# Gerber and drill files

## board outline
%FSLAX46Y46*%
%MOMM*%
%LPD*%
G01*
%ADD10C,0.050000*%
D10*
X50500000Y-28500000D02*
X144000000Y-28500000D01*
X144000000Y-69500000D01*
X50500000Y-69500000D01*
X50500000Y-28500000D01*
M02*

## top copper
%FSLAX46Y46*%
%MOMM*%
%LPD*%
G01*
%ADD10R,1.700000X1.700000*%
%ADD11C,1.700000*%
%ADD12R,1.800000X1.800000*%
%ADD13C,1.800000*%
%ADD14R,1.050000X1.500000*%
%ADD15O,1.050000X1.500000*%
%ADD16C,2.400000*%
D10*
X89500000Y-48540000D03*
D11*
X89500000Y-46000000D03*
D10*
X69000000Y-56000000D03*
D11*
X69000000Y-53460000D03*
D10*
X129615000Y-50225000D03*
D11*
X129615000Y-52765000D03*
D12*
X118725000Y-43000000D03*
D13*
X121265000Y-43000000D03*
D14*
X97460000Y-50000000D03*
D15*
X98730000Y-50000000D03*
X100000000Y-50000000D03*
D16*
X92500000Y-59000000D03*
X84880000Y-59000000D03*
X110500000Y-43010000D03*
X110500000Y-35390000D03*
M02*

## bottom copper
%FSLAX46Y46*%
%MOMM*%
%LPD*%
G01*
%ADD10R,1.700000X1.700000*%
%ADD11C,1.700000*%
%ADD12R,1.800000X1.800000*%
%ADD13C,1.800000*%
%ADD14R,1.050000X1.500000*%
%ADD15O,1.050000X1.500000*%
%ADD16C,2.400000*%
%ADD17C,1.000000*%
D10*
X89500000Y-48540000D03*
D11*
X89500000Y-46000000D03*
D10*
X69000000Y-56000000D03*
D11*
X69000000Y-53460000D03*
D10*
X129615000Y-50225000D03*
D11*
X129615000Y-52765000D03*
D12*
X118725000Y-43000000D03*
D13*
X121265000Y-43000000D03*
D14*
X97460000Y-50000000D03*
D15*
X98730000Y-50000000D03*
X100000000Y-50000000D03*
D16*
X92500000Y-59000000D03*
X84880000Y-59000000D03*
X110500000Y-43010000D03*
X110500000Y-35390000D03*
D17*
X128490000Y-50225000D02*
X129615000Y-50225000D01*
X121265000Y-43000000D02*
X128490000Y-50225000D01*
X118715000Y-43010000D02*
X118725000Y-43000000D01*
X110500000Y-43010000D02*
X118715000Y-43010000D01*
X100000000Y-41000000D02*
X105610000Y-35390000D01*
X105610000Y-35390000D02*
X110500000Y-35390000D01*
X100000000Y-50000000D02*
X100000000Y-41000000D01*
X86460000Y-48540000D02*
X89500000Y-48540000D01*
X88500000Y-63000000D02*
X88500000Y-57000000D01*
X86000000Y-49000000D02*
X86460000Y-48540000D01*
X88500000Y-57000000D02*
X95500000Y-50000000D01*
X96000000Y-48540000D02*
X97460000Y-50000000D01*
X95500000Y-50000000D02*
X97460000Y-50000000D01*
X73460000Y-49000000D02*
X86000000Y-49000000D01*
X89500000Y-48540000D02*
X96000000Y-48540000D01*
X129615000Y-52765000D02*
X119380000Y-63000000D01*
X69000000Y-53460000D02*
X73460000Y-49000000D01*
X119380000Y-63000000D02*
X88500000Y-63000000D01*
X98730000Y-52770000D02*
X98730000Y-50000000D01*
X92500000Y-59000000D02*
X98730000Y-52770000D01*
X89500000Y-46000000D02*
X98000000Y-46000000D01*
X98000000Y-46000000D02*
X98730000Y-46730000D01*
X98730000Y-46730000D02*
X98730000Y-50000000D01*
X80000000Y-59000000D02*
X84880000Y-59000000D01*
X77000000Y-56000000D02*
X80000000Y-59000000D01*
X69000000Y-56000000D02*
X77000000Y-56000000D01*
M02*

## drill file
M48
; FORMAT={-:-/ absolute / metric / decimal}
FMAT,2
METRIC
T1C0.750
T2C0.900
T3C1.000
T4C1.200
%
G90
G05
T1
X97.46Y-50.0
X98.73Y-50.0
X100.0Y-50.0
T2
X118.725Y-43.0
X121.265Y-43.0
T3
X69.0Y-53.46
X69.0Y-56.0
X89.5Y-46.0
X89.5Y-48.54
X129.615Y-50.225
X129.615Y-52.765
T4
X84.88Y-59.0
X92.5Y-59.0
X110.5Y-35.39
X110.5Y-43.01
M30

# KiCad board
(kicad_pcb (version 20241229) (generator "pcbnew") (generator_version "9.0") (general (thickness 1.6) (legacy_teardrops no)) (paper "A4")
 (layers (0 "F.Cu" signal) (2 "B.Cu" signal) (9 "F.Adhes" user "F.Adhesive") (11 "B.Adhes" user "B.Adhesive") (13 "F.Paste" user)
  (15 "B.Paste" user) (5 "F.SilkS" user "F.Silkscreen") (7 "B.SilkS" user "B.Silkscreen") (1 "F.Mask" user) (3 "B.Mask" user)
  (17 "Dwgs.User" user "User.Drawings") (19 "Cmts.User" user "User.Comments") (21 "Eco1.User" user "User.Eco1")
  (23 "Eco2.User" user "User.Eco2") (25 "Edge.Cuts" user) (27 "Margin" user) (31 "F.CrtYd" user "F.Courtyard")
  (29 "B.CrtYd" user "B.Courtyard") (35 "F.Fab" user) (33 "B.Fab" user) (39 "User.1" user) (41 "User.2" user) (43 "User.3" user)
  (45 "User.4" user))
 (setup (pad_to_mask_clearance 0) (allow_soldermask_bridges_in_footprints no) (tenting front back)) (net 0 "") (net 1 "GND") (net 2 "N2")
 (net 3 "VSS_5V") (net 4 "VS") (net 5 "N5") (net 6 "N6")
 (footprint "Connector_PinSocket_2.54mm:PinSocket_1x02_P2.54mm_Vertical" (layer "F.Cu") (at 89.5 48.54 180)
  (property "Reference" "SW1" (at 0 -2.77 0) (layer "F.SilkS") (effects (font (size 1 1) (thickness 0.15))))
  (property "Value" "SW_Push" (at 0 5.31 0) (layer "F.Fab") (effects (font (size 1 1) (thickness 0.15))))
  (pad "1" thru_hole rect (at 0 0 180) (size 1.7 1.7) (drill 1) (layers "*.Cu" "*.Mask") (remove_unused_layers no) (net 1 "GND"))
  (pad "2" thru_hole circle (at 0 2.54 180) (size 1.7 1.7) (drill 1) (layers "*.Cu" "*.Mask") (remove_unused_layers no) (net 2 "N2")))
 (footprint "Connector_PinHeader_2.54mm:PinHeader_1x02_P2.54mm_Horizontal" (layer "F.Cu") (at 69 56 180)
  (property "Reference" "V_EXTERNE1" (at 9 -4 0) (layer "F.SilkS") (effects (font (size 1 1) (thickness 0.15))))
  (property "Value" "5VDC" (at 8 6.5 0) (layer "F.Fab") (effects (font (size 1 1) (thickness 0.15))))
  (pad "1" thru_hole rect (at 0 0 180) (size 1.7 1.7) (drill 1) (layers "*.Cu" "*.Mask") (remove_unused_layers no) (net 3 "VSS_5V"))
  (pad "2" thru_hole circle (at 0 2.54 180) (size 1.7 1.7) (drill 1) (layers "*.Cu" "*.Mask") (remove_unused_layers no) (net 1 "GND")))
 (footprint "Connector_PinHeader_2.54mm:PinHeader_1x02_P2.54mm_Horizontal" (layer "F.Cu") (at 129.615 50.225)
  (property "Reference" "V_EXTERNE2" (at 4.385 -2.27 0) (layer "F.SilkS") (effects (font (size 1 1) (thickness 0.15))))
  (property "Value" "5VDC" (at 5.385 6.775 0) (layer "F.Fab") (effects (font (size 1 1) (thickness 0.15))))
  (pad "1" thru_hole rect (at 0 0) (size 1.7 1.7) (drill 1) (layers "*.Cu" "*.Mask") (remove_unused_layers no) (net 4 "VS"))
  (pad "2" thru_hole circle (at 0 2.54) (size 1.7 1.7) (drill 1) (layers "*.Cu" "*.Mask") (remove_unused_layers no) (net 1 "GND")))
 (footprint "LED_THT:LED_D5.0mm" (layer "F.Cu") (at 118.725 43)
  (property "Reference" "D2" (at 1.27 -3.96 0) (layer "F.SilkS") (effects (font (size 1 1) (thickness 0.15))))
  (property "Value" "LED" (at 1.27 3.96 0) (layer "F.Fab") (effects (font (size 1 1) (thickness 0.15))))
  (pad "1" thru_hole rect (at 0 0) (size 1.8 1.8) (drill 0.9) (layers "*.Cu" "*.Mask") (remove_unused_layers no) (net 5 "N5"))
  (pad "2" thru_hole circle (at 2.54 0) (size 1.8 1.8) (drill 0.9) (layers "*.Cu" "*.Mask") (remove_unused_layers no) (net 4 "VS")))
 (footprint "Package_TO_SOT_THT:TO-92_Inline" (layer "F.Cu") (at 97.46 50)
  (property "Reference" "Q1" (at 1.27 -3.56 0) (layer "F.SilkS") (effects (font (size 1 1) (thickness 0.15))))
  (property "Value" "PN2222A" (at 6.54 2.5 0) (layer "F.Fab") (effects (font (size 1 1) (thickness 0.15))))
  (pad "1" thru_hole rect (at 0 0) (size 1.05 1.5) (drill 0.75) (layers "*.Cu" "*.Mask") (remove_unused_layers no) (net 1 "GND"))
  (pad "2" thru_hole oval (at 1.27 0) (size 1.05 1.5) (drill 0.75) (layers "*.Cu" "*.Mask") (remove_unused_layers no) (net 2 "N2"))
  (pad "3" thru_hole oval (at 2.54 0) (size 1.05 1.5) (drill 0.75) (layers "*.Cu" "*.Mask") (remove_unused_layers no) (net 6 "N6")))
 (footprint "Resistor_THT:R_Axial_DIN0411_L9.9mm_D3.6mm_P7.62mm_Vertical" (layer "F.Cu") (at 92.5 59 180)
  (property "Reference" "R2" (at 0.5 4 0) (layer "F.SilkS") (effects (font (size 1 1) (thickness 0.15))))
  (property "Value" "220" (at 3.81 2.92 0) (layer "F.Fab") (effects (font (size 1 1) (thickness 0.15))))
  (pad "1" thru_hole circle (at 0 0 180) (size 2.4 2.4) (drill 1.2) (layers "*.Cu" "*.Mask") (remove_unused_layers no) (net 2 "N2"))
  (pad "2" thru_hole circle (at 7.62 0 180) (size 2.4 2.4) (drill 1.2) (layers "*.Cu" "*.Mask") (remove_unused_layers no) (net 3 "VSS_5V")))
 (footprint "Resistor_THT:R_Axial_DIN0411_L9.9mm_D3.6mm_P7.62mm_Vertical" (layer "F.Cu") (at 110.5 43.01 90)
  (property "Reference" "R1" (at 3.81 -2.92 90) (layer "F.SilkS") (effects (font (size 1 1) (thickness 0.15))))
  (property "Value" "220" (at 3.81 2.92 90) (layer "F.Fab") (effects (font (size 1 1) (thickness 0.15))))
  (pad "1" thru_hole circle (at 0 0 90) (size 2.4 2.4) (drill 1.2) (layers "*.Cu" "*.Mask") (remove_unused_layers no) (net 5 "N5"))
  (pad "2" thru_hole circle (at 7.62 0 90) (size 2.4 2.4) (drill 1.2) (layers "*.Cu" "*.Mask") (remove_unused_layers no) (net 6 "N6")))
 (gr_rect (start 50.5 28.5) (end 144 69.5) (stroke (width 0.05) (type default)) (fill no) (layer "Edge.Cuts"))
 (segment (start 128.49 50.225) (end 129.615 50.225) (width 1) (layer "B.Cu") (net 4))
 (segment (start 121.265 43) (end 128.49 50.225) (width 1) (layer "B.Cu") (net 4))
 (segment (start 118.715 43.01) (end 118.725 43) (width 1) (layer "B.Cu") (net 5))
 (segment (start 110.5 43.01) (end 118.715 43.01) (width 1) (layer "B.Cu") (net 5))
 (segment (start 100 41) (end 105.61 35.39) (width 1) (layer "B.Cu") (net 6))
 (segment (start 105.61 35.39) (end 110.5 35.39) (width 1) (layer "B.Cu") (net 6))
 (segment (start 100 50) (end 100 41) (width 1) (layer "B.Cu") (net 6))
 (segment (start 86.46 48.54) (end 89.5 48.54) (width 1) (layer "B.Cu") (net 1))
 (segment (start 88.5 63) (end 88.5 57) (width 1) (layer "B.Cu") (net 1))
 (segment (start 86 49) (end 86.46 48.54) (width 1) (layer "B.Cu") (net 1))
 (segment (start 88.5 57) (end 95.5 50) (width 1) (layer "B.Cu") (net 1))
 (segment (start 96 48.54) (end 97.46 50) (width 1) (layer "B.Cu") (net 1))
 (segment (start 95.5 50) (end 97.46 50) (width 1) (layer "B.Cu") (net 1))
 (segment (start 73.46 49) (end 86 49) (width 1) (layer "B.Cu") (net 1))
 (segment (start 89.5 48.54) (end 96 48.54) (width 1) (layer "B.Cu") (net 1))
 (segment (start 129.615 52.765) (end 119.38 63) (width 1) (layer "B.Cu") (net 1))
 (segment (start 69 53.46) (end 73.46 49) (width 1) (layer "B.Cu") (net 1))
 (segment (start 119.38 63) (end 88.5 63) (width 1) (layer "B.Cu") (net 1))
 (segment (start 98.73 52.77) (end 98.73 50) (width 1) (layer "B.Cu") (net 2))
 (segment (start 92.5 59) (end 98.73 52.77) (width 1) (layer "B.Cu") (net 2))
 (segment (start 89.5 46) (end 98 46) (width 1) (layer "B.Cu") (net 2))
 (segment (start 98 46) (end 98.73 46.73) (width 1) (layer "B.Cu") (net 2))
 (segment (start 98.73 46.73) (end 98.73 50) (width 1) (layer "B.Cu") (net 2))
 (segment (start 80 59) (end 84.88 59) (width 1) (layer "B.Cu") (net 3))
 (segment (start 77 56) (end 80 59) (width 1) (layer "B.Cu") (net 3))
 (segment (start 69 56) (end 77 56) (width 1) (layer "B.Cu") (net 3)))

